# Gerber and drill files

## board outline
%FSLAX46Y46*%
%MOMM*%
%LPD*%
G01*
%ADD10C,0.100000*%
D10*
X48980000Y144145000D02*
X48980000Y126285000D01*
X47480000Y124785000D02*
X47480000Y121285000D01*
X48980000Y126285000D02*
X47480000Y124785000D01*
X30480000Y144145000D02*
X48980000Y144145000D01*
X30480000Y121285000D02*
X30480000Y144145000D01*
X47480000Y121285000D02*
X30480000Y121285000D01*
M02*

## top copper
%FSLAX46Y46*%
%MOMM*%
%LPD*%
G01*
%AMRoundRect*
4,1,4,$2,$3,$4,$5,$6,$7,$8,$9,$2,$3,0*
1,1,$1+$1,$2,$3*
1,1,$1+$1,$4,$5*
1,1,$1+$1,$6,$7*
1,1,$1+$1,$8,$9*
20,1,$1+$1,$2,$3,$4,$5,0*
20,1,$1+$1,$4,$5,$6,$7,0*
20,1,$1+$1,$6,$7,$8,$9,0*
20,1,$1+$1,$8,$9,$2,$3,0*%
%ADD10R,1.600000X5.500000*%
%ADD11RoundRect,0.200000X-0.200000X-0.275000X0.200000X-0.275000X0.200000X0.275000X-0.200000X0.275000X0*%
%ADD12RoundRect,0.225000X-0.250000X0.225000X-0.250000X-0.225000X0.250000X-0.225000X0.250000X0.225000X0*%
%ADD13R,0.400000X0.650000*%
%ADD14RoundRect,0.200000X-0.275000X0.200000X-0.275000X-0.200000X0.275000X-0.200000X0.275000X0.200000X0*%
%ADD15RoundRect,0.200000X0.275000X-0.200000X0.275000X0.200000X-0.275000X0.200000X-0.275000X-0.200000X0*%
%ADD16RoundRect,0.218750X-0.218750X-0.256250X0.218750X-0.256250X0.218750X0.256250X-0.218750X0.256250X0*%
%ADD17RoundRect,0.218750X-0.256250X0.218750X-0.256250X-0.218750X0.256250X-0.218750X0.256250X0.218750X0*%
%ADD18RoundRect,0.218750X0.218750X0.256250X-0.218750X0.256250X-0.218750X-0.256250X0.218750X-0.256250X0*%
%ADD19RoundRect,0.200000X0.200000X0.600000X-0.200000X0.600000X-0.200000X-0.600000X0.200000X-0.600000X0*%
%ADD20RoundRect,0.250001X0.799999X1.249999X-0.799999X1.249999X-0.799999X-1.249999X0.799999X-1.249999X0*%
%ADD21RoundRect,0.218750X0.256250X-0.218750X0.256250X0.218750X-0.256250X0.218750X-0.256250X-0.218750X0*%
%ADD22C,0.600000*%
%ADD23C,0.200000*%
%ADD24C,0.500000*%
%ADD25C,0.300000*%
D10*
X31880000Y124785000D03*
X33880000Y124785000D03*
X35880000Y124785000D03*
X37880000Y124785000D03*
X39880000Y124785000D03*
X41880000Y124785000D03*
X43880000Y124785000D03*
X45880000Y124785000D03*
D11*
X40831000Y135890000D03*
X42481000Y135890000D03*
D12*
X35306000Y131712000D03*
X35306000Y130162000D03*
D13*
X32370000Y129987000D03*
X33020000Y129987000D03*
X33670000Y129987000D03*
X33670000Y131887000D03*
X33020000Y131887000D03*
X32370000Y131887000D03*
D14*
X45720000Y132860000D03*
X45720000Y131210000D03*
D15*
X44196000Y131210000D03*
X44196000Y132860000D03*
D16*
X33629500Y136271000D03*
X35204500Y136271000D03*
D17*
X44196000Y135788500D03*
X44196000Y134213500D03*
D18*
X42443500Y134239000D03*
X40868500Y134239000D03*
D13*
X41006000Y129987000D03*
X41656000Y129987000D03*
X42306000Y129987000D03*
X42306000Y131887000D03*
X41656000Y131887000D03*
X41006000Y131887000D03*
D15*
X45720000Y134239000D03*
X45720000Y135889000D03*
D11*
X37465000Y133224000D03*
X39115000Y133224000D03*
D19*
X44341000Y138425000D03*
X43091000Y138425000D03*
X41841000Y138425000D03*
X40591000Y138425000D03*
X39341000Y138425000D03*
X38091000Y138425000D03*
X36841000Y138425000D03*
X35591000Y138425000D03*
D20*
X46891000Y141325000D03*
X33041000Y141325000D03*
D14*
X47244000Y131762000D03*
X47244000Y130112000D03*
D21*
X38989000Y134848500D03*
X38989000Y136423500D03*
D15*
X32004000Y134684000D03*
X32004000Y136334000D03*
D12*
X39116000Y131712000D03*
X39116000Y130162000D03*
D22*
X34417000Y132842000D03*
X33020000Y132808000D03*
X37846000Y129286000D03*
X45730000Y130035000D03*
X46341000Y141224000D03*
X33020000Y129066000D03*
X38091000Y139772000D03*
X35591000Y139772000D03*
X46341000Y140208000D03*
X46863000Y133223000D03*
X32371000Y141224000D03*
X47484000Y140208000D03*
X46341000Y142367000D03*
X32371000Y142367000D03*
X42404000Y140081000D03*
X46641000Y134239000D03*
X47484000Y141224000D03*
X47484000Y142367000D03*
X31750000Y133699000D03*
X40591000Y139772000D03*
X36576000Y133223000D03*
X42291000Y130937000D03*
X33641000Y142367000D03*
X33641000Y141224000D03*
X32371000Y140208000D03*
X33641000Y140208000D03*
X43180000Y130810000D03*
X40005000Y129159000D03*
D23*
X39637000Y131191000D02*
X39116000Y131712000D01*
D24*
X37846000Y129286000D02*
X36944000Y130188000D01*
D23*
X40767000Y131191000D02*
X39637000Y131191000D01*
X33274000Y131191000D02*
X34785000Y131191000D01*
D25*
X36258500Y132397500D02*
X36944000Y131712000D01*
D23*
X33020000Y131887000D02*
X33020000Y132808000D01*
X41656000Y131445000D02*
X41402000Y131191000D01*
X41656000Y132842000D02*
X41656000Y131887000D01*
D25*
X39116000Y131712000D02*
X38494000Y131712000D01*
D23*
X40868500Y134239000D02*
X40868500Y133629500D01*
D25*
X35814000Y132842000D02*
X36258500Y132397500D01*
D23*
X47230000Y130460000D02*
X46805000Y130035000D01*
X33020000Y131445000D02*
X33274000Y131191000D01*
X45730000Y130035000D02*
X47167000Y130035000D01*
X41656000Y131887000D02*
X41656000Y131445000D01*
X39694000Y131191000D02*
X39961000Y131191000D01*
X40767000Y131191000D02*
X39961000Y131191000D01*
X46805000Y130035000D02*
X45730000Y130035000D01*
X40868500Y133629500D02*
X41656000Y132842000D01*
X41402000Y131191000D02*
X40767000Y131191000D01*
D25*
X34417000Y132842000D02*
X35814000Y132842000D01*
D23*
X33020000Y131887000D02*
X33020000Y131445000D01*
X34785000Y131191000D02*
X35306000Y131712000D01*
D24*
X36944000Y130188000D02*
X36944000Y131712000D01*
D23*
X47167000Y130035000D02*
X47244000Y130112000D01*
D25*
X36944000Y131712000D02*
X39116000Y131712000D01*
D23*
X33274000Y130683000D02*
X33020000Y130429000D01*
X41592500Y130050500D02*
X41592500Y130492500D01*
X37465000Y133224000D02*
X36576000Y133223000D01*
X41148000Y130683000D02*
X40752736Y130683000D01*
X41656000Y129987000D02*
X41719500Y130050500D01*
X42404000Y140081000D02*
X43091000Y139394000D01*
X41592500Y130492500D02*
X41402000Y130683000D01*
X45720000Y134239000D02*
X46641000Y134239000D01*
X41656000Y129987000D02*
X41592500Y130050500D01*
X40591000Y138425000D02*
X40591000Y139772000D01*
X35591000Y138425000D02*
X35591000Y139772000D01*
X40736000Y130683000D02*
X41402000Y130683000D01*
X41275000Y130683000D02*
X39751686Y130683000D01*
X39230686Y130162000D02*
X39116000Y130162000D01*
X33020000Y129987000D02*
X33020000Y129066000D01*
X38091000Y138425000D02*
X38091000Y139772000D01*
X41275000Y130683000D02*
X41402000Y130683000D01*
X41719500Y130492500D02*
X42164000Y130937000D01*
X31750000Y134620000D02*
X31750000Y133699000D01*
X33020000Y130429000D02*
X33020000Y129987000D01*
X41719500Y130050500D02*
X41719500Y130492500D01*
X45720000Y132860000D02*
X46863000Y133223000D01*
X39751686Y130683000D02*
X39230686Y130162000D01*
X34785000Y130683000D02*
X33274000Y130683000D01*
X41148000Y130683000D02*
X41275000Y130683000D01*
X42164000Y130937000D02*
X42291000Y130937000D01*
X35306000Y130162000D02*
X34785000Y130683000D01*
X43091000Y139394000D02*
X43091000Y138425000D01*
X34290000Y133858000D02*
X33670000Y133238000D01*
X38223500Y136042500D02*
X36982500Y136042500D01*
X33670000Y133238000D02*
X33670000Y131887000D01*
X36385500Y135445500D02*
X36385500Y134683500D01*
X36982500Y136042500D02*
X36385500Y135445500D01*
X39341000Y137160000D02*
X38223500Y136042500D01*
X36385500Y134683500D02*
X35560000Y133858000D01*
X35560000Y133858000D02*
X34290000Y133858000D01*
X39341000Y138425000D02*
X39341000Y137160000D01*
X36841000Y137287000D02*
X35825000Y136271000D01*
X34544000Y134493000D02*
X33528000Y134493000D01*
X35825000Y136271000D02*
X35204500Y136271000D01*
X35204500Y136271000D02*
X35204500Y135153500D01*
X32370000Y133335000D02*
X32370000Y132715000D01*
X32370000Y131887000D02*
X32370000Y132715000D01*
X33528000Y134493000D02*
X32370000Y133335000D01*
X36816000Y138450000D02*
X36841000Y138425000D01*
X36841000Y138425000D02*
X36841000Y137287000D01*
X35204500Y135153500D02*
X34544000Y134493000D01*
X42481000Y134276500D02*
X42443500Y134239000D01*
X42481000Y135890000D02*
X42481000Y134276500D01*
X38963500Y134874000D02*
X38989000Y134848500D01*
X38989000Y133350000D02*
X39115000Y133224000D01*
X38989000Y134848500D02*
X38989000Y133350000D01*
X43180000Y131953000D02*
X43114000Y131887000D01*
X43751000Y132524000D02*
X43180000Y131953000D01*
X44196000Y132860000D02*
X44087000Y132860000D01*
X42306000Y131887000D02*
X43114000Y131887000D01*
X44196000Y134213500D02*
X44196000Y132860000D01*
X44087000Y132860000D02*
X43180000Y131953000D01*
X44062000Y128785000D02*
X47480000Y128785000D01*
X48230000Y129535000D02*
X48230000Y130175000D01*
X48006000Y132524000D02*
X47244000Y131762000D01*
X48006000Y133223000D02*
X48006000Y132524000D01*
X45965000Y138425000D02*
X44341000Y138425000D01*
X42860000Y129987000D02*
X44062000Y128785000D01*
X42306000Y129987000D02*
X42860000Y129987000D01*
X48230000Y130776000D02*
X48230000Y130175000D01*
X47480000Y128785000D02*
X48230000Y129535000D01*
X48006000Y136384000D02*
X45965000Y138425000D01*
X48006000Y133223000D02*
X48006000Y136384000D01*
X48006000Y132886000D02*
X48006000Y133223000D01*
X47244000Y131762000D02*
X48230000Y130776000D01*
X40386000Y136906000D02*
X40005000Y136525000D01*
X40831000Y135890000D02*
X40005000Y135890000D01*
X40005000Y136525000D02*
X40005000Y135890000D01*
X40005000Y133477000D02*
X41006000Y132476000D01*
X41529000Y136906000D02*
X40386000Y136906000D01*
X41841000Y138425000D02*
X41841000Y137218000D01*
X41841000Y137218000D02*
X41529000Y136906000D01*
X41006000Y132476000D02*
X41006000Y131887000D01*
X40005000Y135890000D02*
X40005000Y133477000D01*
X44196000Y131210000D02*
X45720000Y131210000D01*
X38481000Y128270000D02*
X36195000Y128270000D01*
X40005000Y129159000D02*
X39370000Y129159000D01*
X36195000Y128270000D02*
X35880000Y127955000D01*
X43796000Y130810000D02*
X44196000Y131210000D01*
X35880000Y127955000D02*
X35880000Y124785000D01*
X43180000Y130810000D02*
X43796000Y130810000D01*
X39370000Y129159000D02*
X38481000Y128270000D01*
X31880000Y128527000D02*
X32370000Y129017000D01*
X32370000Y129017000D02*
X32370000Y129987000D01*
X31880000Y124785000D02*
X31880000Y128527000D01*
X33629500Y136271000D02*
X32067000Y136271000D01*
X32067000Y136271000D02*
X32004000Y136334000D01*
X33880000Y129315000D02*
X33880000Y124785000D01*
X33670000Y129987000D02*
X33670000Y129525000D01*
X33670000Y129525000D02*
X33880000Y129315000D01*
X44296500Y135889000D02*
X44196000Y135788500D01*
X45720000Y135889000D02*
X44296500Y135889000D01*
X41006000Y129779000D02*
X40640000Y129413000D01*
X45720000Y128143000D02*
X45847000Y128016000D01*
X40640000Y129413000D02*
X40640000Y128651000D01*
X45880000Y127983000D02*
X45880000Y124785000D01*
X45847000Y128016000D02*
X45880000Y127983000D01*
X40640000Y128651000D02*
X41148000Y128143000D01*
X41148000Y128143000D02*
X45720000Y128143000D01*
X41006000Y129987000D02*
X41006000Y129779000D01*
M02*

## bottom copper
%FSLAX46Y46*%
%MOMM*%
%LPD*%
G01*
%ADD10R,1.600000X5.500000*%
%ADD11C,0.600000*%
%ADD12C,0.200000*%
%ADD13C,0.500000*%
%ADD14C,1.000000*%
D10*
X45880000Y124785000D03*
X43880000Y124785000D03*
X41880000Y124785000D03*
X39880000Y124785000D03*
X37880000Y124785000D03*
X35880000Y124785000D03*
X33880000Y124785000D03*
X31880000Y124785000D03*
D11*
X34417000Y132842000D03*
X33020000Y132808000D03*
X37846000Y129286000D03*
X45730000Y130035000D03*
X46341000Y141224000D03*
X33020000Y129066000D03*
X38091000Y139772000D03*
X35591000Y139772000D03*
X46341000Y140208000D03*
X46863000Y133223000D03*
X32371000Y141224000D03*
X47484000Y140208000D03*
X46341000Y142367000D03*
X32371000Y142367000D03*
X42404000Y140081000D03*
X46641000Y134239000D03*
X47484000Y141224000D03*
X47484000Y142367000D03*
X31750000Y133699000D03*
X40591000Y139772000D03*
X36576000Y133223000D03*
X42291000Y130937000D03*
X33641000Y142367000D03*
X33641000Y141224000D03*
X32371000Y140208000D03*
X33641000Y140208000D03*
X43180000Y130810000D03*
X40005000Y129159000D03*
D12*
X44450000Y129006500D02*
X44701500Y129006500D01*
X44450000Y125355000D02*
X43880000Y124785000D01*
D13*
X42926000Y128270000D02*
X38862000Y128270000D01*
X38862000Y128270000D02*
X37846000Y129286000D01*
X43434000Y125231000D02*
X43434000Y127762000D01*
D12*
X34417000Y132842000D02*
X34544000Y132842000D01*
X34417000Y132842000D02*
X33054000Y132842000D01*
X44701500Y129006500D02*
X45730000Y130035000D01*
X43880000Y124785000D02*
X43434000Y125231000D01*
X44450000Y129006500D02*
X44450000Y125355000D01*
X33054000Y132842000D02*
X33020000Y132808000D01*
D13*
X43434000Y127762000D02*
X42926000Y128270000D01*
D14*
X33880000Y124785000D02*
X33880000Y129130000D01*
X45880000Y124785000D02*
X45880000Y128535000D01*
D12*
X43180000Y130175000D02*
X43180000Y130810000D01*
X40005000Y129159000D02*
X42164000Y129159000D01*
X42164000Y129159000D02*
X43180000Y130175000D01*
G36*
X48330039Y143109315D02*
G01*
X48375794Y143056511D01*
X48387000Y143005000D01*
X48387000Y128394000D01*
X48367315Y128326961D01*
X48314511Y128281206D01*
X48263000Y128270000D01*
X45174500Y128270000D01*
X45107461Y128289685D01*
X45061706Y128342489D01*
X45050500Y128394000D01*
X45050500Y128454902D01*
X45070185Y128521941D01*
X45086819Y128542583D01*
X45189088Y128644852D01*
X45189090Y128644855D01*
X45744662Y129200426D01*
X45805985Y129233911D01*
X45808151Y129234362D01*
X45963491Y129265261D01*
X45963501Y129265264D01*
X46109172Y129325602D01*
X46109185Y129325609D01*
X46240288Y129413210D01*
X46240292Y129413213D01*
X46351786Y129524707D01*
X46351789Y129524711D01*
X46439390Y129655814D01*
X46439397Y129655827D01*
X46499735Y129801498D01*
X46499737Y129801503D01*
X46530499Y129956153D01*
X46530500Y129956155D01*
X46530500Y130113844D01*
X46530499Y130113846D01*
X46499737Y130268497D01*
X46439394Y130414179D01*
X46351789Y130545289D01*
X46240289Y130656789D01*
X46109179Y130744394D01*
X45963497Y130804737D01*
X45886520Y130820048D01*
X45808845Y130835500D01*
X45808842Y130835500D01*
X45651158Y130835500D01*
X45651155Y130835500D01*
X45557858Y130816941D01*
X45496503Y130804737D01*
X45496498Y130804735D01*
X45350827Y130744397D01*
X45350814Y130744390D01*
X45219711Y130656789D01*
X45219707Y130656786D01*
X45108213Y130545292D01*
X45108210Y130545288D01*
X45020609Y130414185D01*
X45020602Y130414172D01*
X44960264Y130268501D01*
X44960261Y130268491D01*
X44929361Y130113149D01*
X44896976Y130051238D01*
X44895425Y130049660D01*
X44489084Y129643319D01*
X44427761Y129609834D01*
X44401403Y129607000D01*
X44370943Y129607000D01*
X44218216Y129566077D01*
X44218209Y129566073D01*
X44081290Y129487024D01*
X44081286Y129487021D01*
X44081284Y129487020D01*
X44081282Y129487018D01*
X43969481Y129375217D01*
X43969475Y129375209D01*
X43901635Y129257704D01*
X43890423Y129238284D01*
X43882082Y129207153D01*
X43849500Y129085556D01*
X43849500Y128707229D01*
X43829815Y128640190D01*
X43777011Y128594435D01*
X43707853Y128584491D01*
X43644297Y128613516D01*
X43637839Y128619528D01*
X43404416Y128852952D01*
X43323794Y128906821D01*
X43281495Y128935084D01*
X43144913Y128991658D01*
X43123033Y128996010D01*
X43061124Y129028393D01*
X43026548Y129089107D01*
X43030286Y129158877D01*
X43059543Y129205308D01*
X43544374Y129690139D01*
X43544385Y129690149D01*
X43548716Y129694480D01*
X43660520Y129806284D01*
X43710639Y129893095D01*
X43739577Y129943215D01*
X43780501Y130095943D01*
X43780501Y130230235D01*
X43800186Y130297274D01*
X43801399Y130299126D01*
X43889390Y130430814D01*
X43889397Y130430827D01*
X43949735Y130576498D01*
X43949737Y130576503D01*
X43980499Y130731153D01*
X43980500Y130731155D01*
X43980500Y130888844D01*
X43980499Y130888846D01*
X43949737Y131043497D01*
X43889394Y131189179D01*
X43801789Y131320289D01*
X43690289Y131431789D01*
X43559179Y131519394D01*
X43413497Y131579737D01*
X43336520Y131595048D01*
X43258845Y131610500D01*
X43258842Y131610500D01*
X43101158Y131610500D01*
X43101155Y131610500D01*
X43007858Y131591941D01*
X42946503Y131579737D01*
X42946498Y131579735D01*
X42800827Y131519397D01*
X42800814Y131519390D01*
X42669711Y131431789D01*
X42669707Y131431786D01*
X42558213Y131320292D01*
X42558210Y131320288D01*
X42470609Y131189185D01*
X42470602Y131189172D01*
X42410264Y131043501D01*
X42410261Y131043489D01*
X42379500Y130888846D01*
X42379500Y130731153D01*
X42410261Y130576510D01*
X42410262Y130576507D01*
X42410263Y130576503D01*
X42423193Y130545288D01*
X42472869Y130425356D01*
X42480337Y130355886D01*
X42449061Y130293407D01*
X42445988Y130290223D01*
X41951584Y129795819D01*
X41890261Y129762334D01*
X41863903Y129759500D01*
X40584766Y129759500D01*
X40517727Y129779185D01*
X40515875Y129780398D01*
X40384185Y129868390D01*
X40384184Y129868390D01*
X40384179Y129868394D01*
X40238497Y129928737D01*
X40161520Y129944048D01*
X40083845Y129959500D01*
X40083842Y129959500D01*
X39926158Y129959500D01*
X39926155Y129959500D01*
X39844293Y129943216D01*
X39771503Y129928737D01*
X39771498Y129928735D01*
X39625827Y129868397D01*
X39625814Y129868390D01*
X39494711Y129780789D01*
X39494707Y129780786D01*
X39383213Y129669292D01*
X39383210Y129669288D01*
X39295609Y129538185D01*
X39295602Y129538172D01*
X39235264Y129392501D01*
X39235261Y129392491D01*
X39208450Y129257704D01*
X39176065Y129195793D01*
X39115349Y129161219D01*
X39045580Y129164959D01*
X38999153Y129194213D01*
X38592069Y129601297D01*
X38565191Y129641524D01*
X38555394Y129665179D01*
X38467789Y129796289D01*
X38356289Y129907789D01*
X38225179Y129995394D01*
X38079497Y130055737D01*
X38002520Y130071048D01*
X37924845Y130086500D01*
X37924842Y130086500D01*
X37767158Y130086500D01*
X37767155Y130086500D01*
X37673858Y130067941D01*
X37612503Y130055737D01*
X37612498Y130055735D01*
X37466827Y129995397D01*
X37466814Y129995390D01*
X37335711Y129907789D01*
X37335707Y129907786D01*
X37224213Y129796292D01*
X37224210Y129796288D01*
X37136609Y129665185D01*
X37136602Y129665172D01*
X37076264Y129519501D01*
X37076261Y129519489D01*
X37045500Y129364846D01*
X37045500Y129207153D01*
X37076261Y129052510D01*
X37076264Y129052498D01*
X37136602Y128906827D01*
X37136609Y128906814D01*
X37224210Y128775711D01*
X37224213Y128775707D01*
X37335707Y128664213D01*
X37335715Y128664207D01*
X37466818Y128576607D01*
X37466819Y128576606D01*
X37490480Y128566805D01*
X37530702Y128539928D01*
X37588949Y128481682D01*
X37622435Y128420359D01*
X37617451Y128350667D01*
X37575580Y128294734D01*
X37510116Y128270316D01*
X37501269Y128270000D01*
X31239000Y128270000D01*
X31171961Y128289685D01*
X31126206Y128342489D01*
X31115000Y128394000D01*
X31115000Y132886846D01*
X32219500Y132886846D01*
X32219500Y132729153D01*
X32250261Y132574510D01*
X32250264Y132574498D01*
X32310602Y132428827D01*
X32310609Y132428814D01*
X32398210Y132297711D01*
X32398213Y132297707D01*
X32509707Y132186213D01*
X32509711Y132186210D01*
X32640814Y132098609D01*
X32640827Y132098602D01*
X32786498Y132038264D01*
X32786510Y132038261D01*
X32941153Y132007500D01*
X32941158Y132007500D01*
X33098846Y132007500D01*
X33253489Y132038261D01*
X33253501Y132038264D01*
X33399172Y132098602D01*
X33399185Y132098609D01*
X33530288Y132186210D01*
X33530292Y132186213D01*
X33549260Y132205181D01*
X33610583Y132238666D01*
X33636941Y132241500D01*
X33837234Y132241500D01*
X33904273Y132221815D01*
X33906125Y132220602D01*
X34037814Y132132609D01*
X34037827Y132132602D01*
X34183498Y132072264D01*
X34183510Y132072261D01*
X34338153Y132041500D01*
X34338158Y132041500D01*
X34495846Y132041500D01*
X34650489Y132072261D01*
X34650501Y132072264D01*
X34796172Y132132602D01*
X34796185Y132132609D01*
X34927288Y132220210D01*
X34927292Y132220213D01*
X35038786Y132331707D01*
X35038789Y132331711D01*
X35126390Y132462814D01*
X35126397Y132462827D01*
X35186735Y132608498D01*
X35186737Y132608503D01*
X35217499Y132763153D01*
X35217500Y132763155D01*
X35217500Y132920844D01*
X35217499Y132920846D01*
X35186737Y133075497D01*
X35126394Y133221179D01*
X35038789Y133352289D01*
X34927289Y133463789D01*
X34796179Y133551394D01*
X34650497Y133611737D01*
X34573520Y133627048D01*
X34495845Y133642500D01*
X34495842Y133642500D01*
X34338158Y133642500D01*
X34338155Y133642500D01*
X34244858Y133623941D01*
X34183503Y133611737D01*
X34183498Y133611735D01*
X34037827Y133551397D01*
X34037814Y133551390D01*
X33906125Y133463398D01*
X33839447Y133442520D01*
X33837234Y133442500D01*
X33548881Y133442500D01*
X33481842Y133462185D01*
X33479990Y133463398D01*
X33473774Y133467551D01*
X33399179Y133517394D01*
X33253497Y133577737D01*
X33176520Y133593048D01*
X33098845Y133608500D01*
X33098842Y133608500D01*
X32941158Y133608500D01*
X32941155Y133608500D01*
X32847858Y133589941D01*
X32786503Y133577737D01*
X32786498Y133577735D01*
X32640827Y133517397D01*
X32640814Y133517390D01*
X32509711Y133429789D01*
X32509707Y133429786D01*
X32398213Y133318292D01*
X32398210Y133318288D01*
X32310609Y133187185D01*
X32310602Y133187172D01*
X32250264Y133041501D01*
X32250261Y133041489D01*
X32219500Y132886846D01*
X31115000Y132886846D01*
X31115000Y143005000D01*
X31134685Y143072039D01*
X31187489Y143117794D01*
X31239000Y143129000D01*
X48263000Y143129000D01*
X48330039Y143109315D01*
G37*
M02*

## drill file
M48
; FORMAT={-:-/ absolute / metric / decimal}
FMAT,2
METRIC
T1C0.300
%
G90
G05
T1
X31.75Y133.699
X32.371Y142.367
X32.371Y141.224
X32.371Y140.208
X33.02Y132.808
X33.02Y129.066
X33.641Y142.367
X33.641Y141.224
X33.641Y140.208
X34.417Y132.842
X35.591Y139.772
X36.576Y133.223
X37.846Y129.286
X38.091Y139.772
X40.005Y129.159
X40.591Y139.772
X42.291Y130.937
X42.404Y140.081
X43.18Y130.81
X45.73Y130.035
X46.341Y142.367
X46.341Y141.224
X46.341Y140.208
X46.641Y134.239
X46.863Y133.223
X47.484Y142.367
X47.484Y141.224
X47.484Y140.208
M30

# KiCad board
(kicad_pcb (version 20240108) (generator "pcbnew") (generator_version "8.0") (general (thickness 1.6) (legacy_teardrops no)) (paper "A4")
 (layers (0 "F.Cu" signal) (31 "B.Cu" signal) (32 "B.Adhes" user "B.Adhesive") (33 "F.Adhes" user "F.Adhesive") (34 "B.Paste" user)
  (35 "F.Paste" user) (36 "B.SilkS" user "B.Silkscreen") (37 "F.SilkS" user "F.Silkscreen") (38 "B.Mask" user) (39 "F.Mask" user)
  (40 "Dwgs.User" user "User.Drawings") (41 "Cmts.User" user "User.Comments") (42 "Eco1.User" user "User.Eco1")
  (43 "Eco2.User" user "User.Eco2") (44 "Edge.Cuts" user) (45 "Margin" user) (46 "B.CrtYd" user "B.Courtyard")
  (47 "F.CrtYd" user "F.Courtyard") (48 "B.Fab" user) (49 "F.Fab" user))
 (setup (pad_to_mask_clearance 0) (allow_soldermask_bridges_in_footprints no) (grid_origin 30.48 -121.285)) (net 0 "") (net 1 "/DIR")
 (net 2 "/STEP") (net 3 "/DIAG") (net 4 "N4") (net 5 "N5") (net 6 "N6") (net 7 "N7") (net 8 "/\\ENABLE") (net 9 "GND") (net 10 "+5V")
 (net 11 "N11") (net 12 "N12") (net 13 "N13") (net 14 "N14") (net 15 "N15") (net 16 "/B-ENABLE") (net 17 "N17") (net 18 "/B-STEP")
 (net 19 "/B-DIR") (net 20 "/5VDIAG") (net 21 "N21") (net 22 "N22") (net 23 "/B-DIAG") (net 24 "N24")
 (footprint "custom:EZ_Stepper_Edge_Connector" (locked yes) (layer "F.Cu") (at 30.48 -121.285)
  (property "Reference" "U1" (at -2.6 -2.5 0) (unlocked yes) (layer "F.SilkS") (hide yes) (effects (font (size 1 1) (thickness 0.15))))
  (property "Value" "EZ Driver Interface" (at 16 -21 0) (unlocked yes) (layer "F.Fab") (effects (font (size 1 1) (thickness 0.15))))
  (pad "1" smd rect (at 1.4 -3.5) (size 1.6 5.5) (layers "F.Cu" "F.Paste" "F.Mask") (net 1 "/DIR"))
  (pad "2" smd rect (at 3.4 -3.5) (size 1.6 5.5) (layers "F.Cu" "F.Paste" "F.Mask") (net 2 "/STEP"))
  (pad "3" smd rect (at 5.4 -3.5) (size 1.6 5.5) (layers "F.Cu" "F.Paste" "F.Mask") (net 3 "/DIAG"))
  (pad "4" smd rect (at 7.4 -3.5) (size 1.6 5.5) (layers "F.Cu" "F.Paste" "F.Mask") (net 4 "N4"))
  (pad "5" smd rect (at 9.4 -3.5) (size 1.6 5.5) (layers "F.Cu" "F.Paste" "F.Mask") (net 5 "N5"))
  (pad "6" smd rect (at 11.4 -3.5) (size 1.6 5.5) (layers "F.Cu" "F.Paste" "F.Mask") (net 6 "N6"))
  (pad "7" smd rect (at 13.4 -3.5) (size 1.6 5.5) (layers "F.Cu" "F.Paste" "F.Mask") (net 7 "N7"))
  (pad "8" smd rect (at 15.4 -3.5) (size 1.6 5.5) (layers "F.Cu" "F.Paste" "F.Mask") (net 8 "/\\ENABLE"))
  (pad "9" smd rect (at 15.4 -3.5) (size 1.6 5.5) (layers "B.Cu" "B.Paste" "B.Mask") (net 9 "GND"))
  (pad "10" smd rect (at 13.4 -3.5) (size 1.6 5.5) (layers "B.Cu" "B.Paste" "B.Mask") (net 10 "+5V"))
  (pad "11" smd rect (at 11.4 -3.5) (size 1.6 5.5) (layers "B.Cu" "B.Paste" "B.Mask") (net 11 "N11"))
  (pad "12" smd rect (at 9.4 -3.5) (size 1.6 5.5) (layers "B.Cu" "B.Paste" "B.Mask") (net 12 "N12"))
  (pad "13" smd rect (at 7.4 -3.5) (size 1.6 5.5) (layers "B.Cu" "B.Paste" "B.Mask") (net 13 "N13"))
  (pad "14" smd rect (at 5.4 -3.5) (size 1.6 5.5) (layers "B.Cu" "B.Paste" "B.Mask") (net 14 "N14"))
  (pad "15" smd rect (at 3.4 -3.5) (size 1.6 5.5) (layers "B.Cu" "B.Paste" "B.Mask") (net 9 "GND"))
  (pad "16" smd rect (at 1.4 -3.5) (size 1.6 5.5) (layers "B.Cu" "B.Paste" "B.Mask") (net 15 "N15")))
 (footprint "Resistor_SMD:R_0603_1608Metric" (layer "F.Cu") (at 41.656 -135.89)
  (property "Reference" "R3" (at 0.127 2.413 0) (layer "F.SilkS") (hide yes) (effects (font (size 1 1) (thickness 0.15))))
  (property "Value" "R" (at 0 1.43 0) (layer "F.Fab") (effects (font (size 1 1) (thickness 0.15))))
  (pad "1" smd roundrect (at -0.825 0) (size 0.8 0.95) (layers "F.Cu" "F.Paste" "F.Mask") (roundrect_rratio 0.25) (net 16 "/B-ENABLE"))
  (pad "2" smd roundrect (at 0.825 0) (size 0.8 0.95) (layers "F.Cu" "F.Paste" "F.Mask") (roundrect_rratio 0.25) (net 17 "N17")))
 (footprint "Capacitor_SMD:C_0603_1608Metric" (layer "F.Cu") (at 35.306 -130.937 -90)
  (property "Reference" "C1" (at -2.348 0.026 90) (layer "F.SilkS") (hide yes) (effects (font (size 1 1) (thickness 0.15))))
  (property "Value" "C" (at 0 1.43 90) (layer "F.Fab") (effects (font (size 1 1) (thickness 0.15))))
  (pad "1" smd roundrect (at -0.775 0 270) (size 0.9 0.95) (layers "F.Cu" "F.Paste" "F.Mask") (roundrect_rratio 0.25) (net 10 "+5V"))
  (pad "2" smd roundrect (at 0.775 0 270) (size 0.9 0.95) (layers "F.Cu" "F.Paste" "F.Mask") (roundrect_rratio 0.25) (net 9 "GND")))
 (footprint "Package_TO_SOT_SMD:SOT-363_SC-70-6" (layer "F.Cu") (at 33.02 -130.937 90)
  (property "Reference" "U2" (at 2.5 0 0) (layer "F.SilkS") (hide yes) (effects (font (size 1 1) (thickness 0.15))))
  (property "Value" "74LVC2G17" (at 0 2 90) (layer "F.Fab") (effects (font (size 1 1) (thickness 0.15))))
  (pad "1" smd rect (at -0.95 -0.65 90) (size 0.65 0.4) (layers "F.Cu" "F.Paste" "F.Mask") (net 1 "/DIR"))
  (pad "2" smd rect (at -0.95 0 90) (size 0.65 0.4) (layers "F.Cu" "F.Paste" "F.Mask") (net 9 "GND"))
  (pad "3" smd rect (at -0.95 0.65 90) (size 0.65 0.4) (layers "F.Cu" "F.Paste" "F.Mask") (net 2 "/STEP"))
  (pad "4" smd rect (at 0.95 0.65 90) (size 0.65 0.4) (layers "F.Cu" "F.Paste" "F.Mask") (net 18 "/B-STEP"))
  (pad "5" smd rect (at 0.95 0 90) (size 0.65 0.4) (layers "F.Cu" "F.Paste" "F.Mask") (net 10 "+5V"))
  (pad "6" smd rect (at 0.95 -0.65 90) (size 0.65 0.4) (layers "F.Cu" "F.Paste" "F.Mask") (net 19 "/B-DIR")))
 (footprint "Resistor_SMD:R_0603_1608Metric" (layer "F.Cu") (at 45.72 -132.035 -90)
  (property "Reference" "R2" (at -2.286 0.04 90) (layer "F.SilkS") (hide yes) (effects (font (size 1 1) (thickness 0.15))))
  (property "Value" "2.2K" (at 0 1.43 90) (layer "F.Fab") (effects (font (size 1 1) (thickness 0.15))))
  (pad "1" smd roundrect (at -0.825 0 270) (size 0.8 0.95) (layers "F.Cu" "F.Paste" "F.Mask") (roundrect_rratio 0.25) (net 9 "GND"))
  (pad "2" smd roundrect (at 0.825 0 270) (size 0.8 0.95) (layers "F.Cu" "F.Paste" "F.Mask") (roundrect_rratio 0.25) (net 3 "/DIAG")))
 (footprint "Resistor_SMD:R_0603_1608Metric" (layer "F.Cu") (at 44.196 -132.035 90)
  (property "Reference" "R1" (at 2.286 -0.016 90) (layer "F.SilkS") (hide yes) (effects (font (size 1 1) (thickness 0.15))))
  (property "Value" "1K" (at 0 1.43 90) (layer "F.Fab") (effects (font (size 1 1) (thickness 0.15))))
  (pad "1" smd roundrect (at -0.825 0 90) (size 0.8 0.95) (layers "F.Cu" "F.Paste" "F.Mask") (roundrect_rratio 0.25) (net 3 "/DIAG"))
  (pad "2" smd roundrect (at 0.825 0 90) (size 0.8 0.95) (layers "F.Cu" "F.Paste" "F.Mask") (roundrect_rratio 0.25) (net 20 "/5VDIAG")))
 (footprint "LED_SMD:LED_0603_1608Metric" (layer "F.Cu") (at 34.417 -136.271)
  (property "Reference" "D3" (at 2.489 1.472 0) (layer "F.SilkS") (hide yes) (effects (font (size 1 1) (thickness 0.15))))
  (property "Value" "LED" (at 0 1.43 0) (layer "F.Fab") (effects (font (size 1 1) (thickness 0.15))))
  (pad "1" smd roundrect (at -0.7875 0) (size 0.875 0.95) (layers "F.Cu" "F.Paste" "F.Mask") (roundrect_rratio 0.25) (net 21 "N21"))
  (pad "2" smd roundrect (at 0.7875 0) (size 0.875 0.95) (layers "F.Cu" "F.Paste" "F.Mask") (roundrect_rratio 0.25) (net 19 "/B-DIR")))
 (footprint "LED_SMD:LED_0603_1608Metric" (layer "F.Cu") (at 44.196 -135.001 -90)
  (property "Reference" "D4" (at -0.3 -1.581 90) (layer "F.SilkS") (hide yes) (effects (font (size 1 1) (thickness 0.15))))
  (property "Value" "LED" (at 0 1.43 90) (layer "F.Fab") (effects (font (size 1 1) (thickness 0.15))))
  (pad "1" smd roundrect (at -0.7875 0 270) (size 0.875 0.95) (layers "F.Cu" "F.Paste" "F.Mask") (roundrect_rratio 0.25) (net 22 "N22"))
  (pad "2" smd roundrect (at 0.7875 0 270) (size 0.875 0.95) (layers "F.Cu" "F.Paste" "F.Mask") (roundrect_rratio 0.25) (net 20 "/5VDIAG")))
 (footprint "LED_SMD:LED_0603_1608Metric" (layer "F.Cu") (at 41.656 -134.239 180)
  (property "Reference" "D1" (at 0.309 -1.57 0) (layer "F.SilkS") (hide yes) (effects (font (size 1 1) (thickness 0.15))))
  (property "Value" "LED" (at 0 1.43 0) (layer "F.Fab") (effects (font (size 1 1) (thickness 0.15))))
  (pad "1" smd roundrect (at -0.7875 0 180) (size 0.875 0.95) (layers "F.Cu" "F.Paste" "F.Mask") (roundrect_rratio 0.25) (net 17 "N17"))
  (pad "2" smd roundrect (at 0.7875 0 180) (size 0.875 0.95) (layers "F.Cu" "F.Paste" "F.Mask") (roundrect_rratio 0.25) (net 10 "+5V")))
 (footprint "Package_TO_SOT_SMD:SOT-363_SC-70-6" (layer "F.Cu") (at 41.656 -130.937 90)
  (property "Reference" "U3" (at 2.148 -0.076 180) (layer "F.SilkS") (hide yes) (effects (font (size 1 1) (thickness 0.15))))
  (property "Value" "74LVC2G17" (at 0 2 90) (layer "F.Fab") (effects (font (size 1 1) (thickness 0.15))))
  (pad "1" smd rect (at -0.95 -0.65 90) (size 0.65 0.4) (layers "F.Cu" "F.Paste" "F.Mask") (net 8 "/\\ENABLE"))
  (pad "2" smd rect (at -0.95 0 90) (size 0.65 0.4) (layers "F.Cu" "F.Paste" "F.Mask") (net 9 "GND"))
  (pad "3" smd rect (at -0.95 0.65 90) (size 0.65 0.4) (layers "F.Cu" "F.Paste" "F.Mask") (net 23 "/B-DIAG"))
  (pad "4" smd rect (at 0.95 0.65 90) (size 0.65 0.4) (layers "F.Cu" "F.Paste" "F.Mask") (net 20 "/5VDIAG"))
  (pad "5" smd rect (at 0.95 0 90) (size 0.65 0.4) (layers "F.Cu" "F.Paste" "F.Mask") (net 10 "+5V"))
  (pad "6" smd rect (at 0.95 -0.65 90) (size 0.65 0.4) (layers "F.Cu" "F.Paste" "F.Mask") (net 16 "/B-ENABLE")))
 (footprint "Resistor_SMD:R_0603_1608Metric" (layer "F.Cu") (at 45.72 -135.064 90)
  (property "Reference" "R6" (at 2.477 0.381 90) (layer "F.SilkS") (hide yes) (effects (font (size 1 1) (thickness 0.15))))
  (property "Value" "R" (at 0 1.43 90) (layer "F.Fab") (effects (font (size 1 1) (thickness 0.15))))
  (pad "1" smd roundrect (at -0.825 0 90) (size 0.8 0.95) (layers "F.Cu" "F.Paste" "F.Mask") (roundrect_rratio 0.25) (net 9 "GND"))
  (pad "2" smd roundrect (at 0.825 0 90) (size 0.8 0.95) (layers "F.Cu" "F.Paste" "F.Mask") (roundrect_rratio 0.25) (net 22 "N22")))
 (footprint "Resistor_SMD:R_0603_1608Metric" (layer "F.Cu") (at 38.29 -133.224)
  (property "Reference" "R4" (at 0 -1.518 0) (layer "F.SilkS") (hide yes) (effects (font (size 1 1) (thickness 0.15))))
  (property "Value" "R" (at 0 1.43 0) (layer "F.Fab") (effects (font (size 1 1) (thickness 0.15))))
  (pad "1" smd roundrect (at -0.825 0) (size 0.8 0.95) (layers "F.Cu" "F.Paste" "F.Mask") (roundrect_rratio 0.25) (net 9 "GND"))
  (pad "2" smd roundrect (at 0.825 0) (size 0.8 0.95) (layers "F.Cu" "F.Paste" "F.Mask") (roundrect_rratio 0.25) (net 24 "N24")))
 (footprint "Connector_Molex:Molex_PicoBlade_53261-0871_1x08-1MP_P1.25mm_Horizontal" (layer "F.Cu") (at 39.966 -140.825 180)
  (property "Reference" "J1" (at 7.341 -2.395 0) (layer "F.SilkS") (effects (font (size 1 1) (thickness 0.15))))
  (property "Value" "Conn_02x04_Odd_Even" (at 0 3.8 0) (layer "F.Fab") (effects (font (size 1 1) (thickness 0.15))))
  (pad "1" smd roundrect (at -4.375 -2.4 180) (size 0.8 1.6) (layers "F.Cu" "F.Paste" "F.Mask") (roundrect_rratio 0.25) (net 23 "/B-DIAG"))
  (pad "2" smd roundrect (at -3.125 -2.4 180) (size 0.8 1.6) (layers "F.Cu" "F.Paste" "F.Mask") (roundrect_rratio 0.25) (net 9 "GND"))
  (pad "3" smd roundrect (at -1.875 -2.4 180) (size 0.8 1.6) (layers "F.Cu" "F.Paste" "F.Mask") (roundrect_rratio 0.25) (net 16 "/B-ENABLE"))
  (pad "4" smd roundrect (at -0.625 -2.4 180) (size 0.8 1.6) (layers "F.Cu" "F.Paste" "F.Mask") (roundrect_rratio 0.25) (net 9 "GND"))
  (pad "5" smd roundrect (at 0.625 -2.4 180) (size 0.8 1.6) (layers "F.Cu" "F.Paste" "F.Mask") (roundrect_rratio 0.25) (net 18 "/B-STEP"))
  (pad "6" smd roundrect (at 1.875 -2.4 180) (size 0.8 1.6) (layers "F.Cu" "F.Paste" "F.Mask") (roundrect_rratio 0.25) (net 9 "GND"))
  (pad "7" smd roundrect (at 3.125 -2.4 180) (size 0.8 1.6) (layers "F.Cu" "F.Paste" "F.Mask") (roundrect_rratio 0.25) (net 19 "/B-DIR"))
  (pad "8" smd roundrect (at 4.375 -2.4 180) (size 0.8 1.6) (layers "F.Cu" "F.Paste" "F.Mask") (roundrect_rratio 0.25) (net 9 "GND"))
  (pad "MP" smd roundrect (at -6.925 0.5 180) (size 2.1 3) (layers "F.Cu" "F.Paste" "F.Mask") (roundrect_rratio 0.1190480952) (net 9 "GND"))
  (pad "MP" smd roundrect (at 6.925 0.5 180) (size 2.1 3) (layers "F.Cu" "F.Paste" "F.Mask") (roundrect_rratio 0.1190480952) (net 9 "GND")))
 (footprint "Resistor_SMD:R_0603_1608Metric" (layer "F.Cu") (at 47.244 -130.937 -90)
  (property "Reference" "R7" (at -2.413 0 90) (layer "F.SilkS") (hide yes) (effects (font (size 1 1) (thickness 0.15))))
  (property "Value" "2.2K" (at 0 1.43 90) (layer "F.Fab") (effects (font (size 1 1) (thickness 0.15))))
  (pad "1" smd roundrect (at -0.825 0 270) (size 0.8 0.95) (layers "F.Cu" "F.Paste" "F.Mask") (roundrect_rratio 0.25) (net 23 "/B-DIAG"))
  (pad "2" smd roundrect (at 0.825 0 270) (size 0.8 0.95) (layers "F.Cu" "F.Paste" "F.Mask") (roundrect_rratio 0.25) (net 10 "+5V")))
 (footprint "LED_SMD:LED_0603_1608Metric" (layer "F.Cu") (at 38.989 -135.636 90)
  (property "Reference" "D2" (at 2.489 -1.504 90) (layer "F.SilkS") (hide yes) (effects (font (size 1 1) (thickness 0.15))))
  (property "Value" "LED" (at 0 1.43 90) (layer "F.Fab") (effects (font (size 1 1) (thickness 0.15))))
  (pad "1" smd roundrect (at -0.7875 0 90) (size 0.875 0.95) (layers "F.Cu" "F.Paste" "F.Mask") (roundrect_rratio 0.25) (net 24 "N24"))
  (pad "2" smd roundrect (at 0.7875 0 90) (size 0.875 0.95) (layers "F.Cu" "F.Paste" "F.Mask") (roundrect_rratio 0.25) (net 18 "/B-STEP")))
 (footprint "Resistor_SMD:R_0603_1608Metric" (layer "F.Cu") (at 32.004 -135.509 90)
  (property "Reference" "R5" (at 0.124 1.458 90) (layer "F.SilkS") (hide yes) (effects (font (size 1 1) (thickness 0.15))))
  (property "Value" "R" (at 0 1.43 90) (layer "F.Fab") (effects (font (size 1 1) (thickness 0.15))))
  (pad "1" smd roundrect (at -0.825 0 90) (size 0.8 0.95) (layers "F.Cu" "F.Paste" "F.Mask") (roundrect_rratio 0.25) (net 9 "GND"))
  (pad "2" smd roundrect (at 0.825 0 90) (size 0.8 0.95) (layers "F.Cu" "F.Paste" "F.Mask") (roundrect_rratio 0.25) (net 21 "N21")))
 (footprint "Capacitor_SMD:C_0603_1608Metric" (layer "F.Cu") (at 39.116 -130.937 -90)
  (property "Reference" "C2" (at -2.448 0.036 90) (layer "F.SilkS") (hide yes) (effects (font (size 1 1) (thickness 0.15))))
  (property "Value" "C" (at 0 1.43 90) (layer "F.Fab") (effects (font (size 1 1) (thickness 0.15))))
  (pad "1" smd roundrect (at -0.775 0 270) (size 0.9 0.95) (layers "F.Cu" "F.Paste" "F.Mask") (roundrect_rratio 0.25) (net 10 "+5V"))
  (pad "2" smd roundrect (at 0.775 0 270) (size 0.9 0.95) (layers "F.Cu" "F.Paste" "F.Mask") (roundrect_rratio 0.25) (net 9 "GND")))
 (gr_line (start 48.98 -144.145) (end 48.98 -126.285) (stroke (width 0.1) (type default)) (layer "Edge.Cuts"))
 (gr_line (start 47.48 -124.785) (end 47.48 -121.285) (stroke (width 0.1) (type default)) (layer "Edge.Cuts"))
 (gr_line (start 48.98 -126.285) (end 47.48 -124.785) (stroke (width 0.1) (type default)) (layer "Edge.Cuts"))
 (gr_line (start 30.48 -144.145) (end 48.98 -144.145) (stroke (width 0.1) (type default)) (layer "Edge.Cuts"))
 (gr_line (start 30.48 -121.285) (end 30.48 -144.145) (stroke (width 0.1) (type default)) (layer "Edge.Cuts"))
 (gr_line (start 47.48 -121.285) (end 30.48 -121.285) (stroke (width 0.1) (type default)) (layer "Edge.Cuts"))
 (segment (start 39.637 -131.191) (end 39.116 -131.712) (width 0.2) (layer "F.Cu") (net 10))
 (segment (start 37.846 -129.286) (end 36.944 -130.188) (width 0.5) (layer "F.Cu") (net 10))
 (segment (start 40.767 -131.191) (end 39.637 -131.191) (width 0.2) (layer "F.Cu") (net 10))
 (segment (start 33.274 -131.191) (end 34.785 -131.191) (width 0.2) (layer "F.Cu") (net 10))
 (segment (start 36.2585 -132.3975) (end 36.944 -131.712) (width 0.3) (layer "F.Cu") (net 10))
 (segment (start 33.02 -131.887) (end 33.02 -132.808) (width 0.2) (layer "F.Cu") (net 10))
 (segment (start 41.656 -131.445) (end 41.402 -131.191) (width 0.2) (layer "F.Cu") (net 10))
 (segment (start 41.656 -132.842) (end 41.656 -131.887) (width 0.2) (layer "F.Cu") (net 10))
 (segment (start 39.116 -131.712) (end 38.494 -131.712) (width 0.3) (layer "F.Cu") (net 10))
 (segment (start 40.8685 -134.239) (end 40.8685 -133.6295) (width 0.2) (layer "F.Cu") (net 10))
 (segment (start 35.814 -132.842) (end 36.2585 -132.3975) (width 0.3) (layer "F.Cu") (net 10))
 (segment (start 47.23 -130.46) (end 46.805 -130.035) (width 0.2) (layer "F.Cu") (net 10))
 (segment (start 33.02 -131.445) (end 33.274 -131.191) (width 0.2) (layer "F.Cu") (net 10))
 (segment (start 45.73 -130.035) (end 47.167 -130.035) (width 0.2) (layer "F.Cu") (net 10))
 (segment (start 41.656 -131.887) (end 41.656 -131.445) (width 0.2) (layer "F.Cu") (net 10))
 (segment (start 39.694 -131.191) (end 39.961 -131.191) (width 0.2) (layer "F.Cu") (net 10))
 (segment (start 40.767 -131.191) (end 39.961 -131.191) (width 0.2) (layer "F.Cu") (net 10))
 (segment (start 46.805 -130.035) (end 45.73 -130.035) (width 0.2) (layer "F.Cu") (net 10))
 (segment (start 40.8685 -133.6295) (end 41.656 -132.842) (width 0.2) (layer "F.Cu") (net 10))
 (segment (start 41.402 -131.191) (end 40.767 -131.191) (width 0.2) (layer "F.Cu") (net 10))
 (segment (start 34.417 -132.842) (end 35.814 -132.842) (width 0.3) (layer "F.Cu") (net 10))
 (segment (start 33.02 -131.887) (end 33.02 -131.445) (width 0.2) (layer "F.Cu") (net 10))
 (segment (start 34.785 -131.191) (end 35.306 -131.712) (width 0.2) (layer "F.Cu") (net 10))
 (segment (start 36.944 -130.188) (end 36.944 -131.712) (width 0.5) (layer "F.Cu") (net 10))
 (segment (start 47.167 -130.035) (end 47.244 -130.112) (width 0.2) (layer "F.Cu") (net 10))
 (segment (start 36.944 -131.712) (end 39.116 -131.712) (width 0.3) (layer "F.Cu") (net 10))
 (via (at 34.417 -132.842) (size 0.6) (drill 0.3) (layers "F.Cu" "B.Cu") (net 10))
 (via (at 33.02 -132.808) (size 0.6) (drill 0.3) (layers "F.Cu" "B.Cu") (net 10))
 (via (at 37.846 -129.286) (size 0.6) (drill 0.3) (layers "F.Cu" "B.Cu") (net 10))
 (via (at 45.73 -130.035) (size 0.6) (drill 0.3) (layers "F.Cu" "B.Cu") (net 10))
 (segment (start 44.45 -129.0065) (end 44.7015 -129.0065) (width 0.2) (layer "B.Cu") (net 10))
 (segment (start 44.45 -125.355) (end 43.88 -124.785) (width 0.2) (layer "B.Cu") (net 10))
 (segment (start 42.926 -128.27) (end 38.862 -128.27) (width 0.5) (layer "B.Cu") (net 10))
 (segment (start 38.862 -128.27) (end 37.846 -129.286) (width 0.5) (layer "B.Cu") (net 10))
 (segment (start 43.434 -125.231) (end 43.434 -127.762) (width 0.5) (layer "B.Cu") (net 10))
 (segment (start 34.417 -132.842) (end 34.544 -132.842) (width 0.2) (layer "B.Cu") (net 10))
 (segment (start 34.417 -132.842) (end 33.054 -132.842) (width 0.2) (layer "B.Cu") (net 10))
 (segment (start 44.7015 -129.0065) (end 45.73 -130.035) (width 0.2) (layer "B.Cu") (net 10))
 (segment (start 43.88 -124.785) (end 43.434 -125.231) (width 0.2) (layer "B.Cu") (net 10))
 (segment (start 44.45 -129.0065) (end 44.45 -125.355) (width 0.2) (layer "B.Cu") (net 10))
 (segment (start 33.054 -132.842) (end 33.02 -132.808) (width 0.2) (layer "B.Cu") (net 10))
 (segment (start 43.434 -127.762) (end 42.926 -128.27) (width 0.5) (layer "B.Cu") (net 10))
 (segment (start 33.274 -130.683) (end 33.02 -130.429) (width 0.2) (layer "F.Cu") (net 9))
 (segment (start 41.5925 -130.0505) (end 41.5925 -130.4925) (width 0.2) (layer "F.Cu") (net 9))
 (segment (start 37.465 -133.224) (end 36.576 -133.223) (width 0.2) (layer "F.Cu") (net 9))
 (segment (start 41.148 -130.683) (end 40.752736 -130.683) (width 0.2) (layer "F.Cu") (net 9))
 (segment (start 41.656 -129.987) (end 41.7195 -130.0505) (width 0.2) (layer "F.Cu") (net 9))
 (segment (start 42.404 -140.081) (end 43.091 -139.394) (width 0.2) (layer "F.Cu") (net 9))
 (segment (start 41.5925 -130.4925) (end 41.402 -130.683) (width 0.2) (layer "F.Cu") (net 9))
 (segment (start 45.72 -134.239) (end 46.641 -134.239) (width 0.2) (layer "F.Cu") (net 9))
 (segment (start 41.656 -129.987) (end 41.5925 -130.0505) (width 0.2) (layer "F.Cu") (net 9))
 (segment (start 40.591 -138.425) (end 40.591 -139.772) (width 0.2) (layer "F.Cu") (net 9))
 (segment (start 35.591 -138.425) (end 35.591 -139.772) (width 0.2) (layer "F.Cu") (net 9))
 (segment (start 40.736 -130.683) (end 41.402 -130.683) (width 0.2) (layer "F.Cu") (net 9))
 (segment (start 41.275 -130.683) (end 39.751686 -130.683) (width 0.2) (layer "F.Cu") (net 9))
 (segment (start 39.230686 -130.162) (end 39.116 -130.162) (width 0.2) (layer "F.Cu") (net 9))
 (segment (start 33.02 -129.987) (end 33.02 -129.066) (width 0.2) (layer "F.Cu") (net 9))
 (segment (start 38.091 -138.425) (end 38.091 -139.772) (width 0.2) (layer "F.Cu") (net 9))
 (segment (start 41.275 -130.683) (end 41.402 -130.683) (width 0.2) (layer "F.Cu") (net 9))
 (segment (start 41.7195 -130.4925) (end 42.164 -130.937) (width 0.2) (layer "F.Cu") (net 9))
 (segment (start 31.75 -134.62) (end 31.75 -133.699) (width 0.2) (layer "F.Cu") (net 9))
 (segment (start 33.02 -130.429) (end 33.02 -129.987) (width 0.2) (layer "F.Cu") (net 9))
 (segment (start 41.7195 -130.0505) (end 41.7195 -130.4925) (width 0.2) (layer "F.Cu") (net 9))
 (segment (start 45.72 -132.86) (end 46.863 -133.223) (width 0.2) (layer "F.Cu") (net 9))
 (segment (start 39.751686 -130.683) (end 39.230686 -130.162) (width 0.2) (layer "F.Cu") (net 9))
 (segment (start 34.785 -130.683) (end 33.274 -130.683) (width 0.2) (layer "F.Cu") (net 9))
 (segment (start 41.148 -130.683) (end 41.275 -130.683) (width 0.2) (layer "F.Cu") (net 9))
 (segment (start 42.164 -130.937) (end 42.291 -130.937) (width 0.2) (layer "F.Cu") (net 9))
 (segment (start 35.306 -130.162) (end 34.785 -130.683) (width 0.2) (layer "F.Cu") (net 9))
 (segment (start 43.091 -139.394) (end 43.091 -138.425) (width 0.2) (layer "F.Cu") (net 9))
 (via (at 46.341 -141.224) (size 0.6) (drill 0.3) (layers "F.Cu" "B.Cu") (free yes) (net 9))
 (via (at 33.02 -129.066) (size 0.6) (drill 0.3) (layers "F.Cu" "B.Cu") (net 9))
 (via (at 38.091 -139.772) (size 0.6) (drill 0.3) (layers "F.Cu" "B.Cu") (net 9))
 (via (at 35.591 -139.772) (size 0.6) (drill 0.3) (layers "F.Cu" "B.Cu") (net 9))
 (via (at 46.341 -140.208) (size 0.6) (drill 0.3) (layers "F.Cu" "B.Cu") (free yes) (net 9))
 (via (at 46.863 -133.223) (size 0.6) (drill 0.3) (layers "F.Cu" "B.Cu") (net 9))
 (via (at 32.371 -141.224) (size 0.6) (drill 0.3) (layers "F.Cu" "B.Cu") (free yes) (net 9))
 (via (at 47.484 -140.208) (size 0.6) (drill 0.3) (layers "F.Cu" "B.Cu") (free yes) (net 9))
 (via (at 46.341 -142.367) (size 0.6) (drill 0.3) (layers "F.Cu" "B.Cu") (free yes) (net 9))
 (via (at 32.371 -142.367) (size 0.6) (drill 0.3) (layers "F.Cu" "B.Cu") (free yes) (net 9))
 (via (at 42.404 -140.081) (size 0.6) (drill 0.3) (layers "F.Cu" "B.Cu") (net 9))
 (via (at 46.641 -134.239) (size 0.6) (drill 0.3) (layers "F.Cu" "B.Cu") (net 9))
 (via (at 47.484 -141.224) (size 0.6) (drill 0.3) (layers "F.Cu" "B.Cu") (free yes) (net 9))
 (via (at 47.484 -142.367) (size 0.6) (drill 0.3) (layers "F.Cu" "B.Cu") (free yes) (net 9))
 (via (at 31.75 -133.699) (size 0.6) (drill 0.3) (layers "F.Cu" "B.Cu") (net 9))
 (via (at 40.591 -139.772) (size 0.6) (drill 0.3) (layers "F.Cu" "B.Cu") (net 9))
 (via (at 36.576 -133.223) (size 0.6) (drill 0.3) (layers "F.Cu" "B.Cu") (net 9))
 (via (at 42.291 -130.937) (size 0.6) (drill 0.3) (layers "F.Cu" "B.Cu") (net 9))
 (via (at 33.641 -142.367) (size 0.6) (drill 0.3) (layers "F.Cu" "B.Cu") (free yes) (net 9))
 (via (at 33.641 -141.224) (size 0.6) (drill 0.3) (layers "F.Cu" "B.Cu") (free yes) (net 9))
 (via (at 32.371 -140.208) (size 0.6) (drill 0.3) (layers "F.Cu" "B.Cu") (free yes) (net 9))
 (via (at 33.641 -140.208) (size 0.6) (drill 0.3) (layers "F.Cu" "B.Cu") (free yes) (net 9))
 (segment (start 33.88 -124.785) (end 33.88 -129.13) (width 1) (layer "B.Cu") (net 9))
 (segment (start 45.88 -124.785) (end 45.88 -128.535) (width 1) (layer "B.Cu") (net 9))
 (segment (start 34.29 -133.858) (end 33.67 -133.238) (width 0.2) (layer "F.Cu") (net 18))
 (segment (start 38.2235 -136.0425) (end 36.9825 -136.0425) (width 0.2) (layer "F.Cu") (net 18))
 (segment (start 33.67 -133.238) (end 33.67 -131.887) (width 0.2) (layer "F.Cu") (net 18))
 (segment (start 36.3855 -135.4455) (end 36.3855 -134.6835) (width 0.2) (layer "F.Cu") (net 18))
 (segment (start 36.9825 -136.0425) (end 36.3855 -135.4455) (width 0.2) (layer "F.Cu") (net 18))
 (segment (start 39.341 -137.16) (end 38.2235 -136.0425) (width 0.2) (layer "F.Cu") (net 18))
 (segment (start 36.3855 -134.6835) (end 35.56 -133.858) (width 0.2) (layer "F.Cu") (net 18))
 (segment (start 35.56 -133.858) (end 34.29 -133.858) (width 0.2) (layer "F.Cu") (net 18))
 (segment (start 39.341 -138.425) (end 39.341 -137.16) (width 0.2) (layer "F.Cu") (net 18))
 (segment (start 36.841 -137.287) (end 35.825 -136.271) (width 0.2) (layer "F.Cu") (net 19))
 (segment (start 34.544 -134.493) (end 33.528 -134.493) (width 0.2) (layer "F.Cu") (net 19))
 (segment (start 35.825 -136.271) (end 35.2045 -136.271) (width 0.2) (layer "F.Cu") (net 19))
 (segment (start 35.2045 -136.271) (end 35.2045 -135.1535) (width 0.2) (layer "F.Cu") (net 19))
 (segment (start 32.37 -133.335) (end 32.37 -132.715) (width 0.2) (layer "F.Cu") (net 19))
 (segment (start 32.37 -131.887) (end 32.37 -132.715) (width 0.2) (layer "F.Cu") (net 19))
 (segment (start 33.528 -134.493) (end 32.37 -133.335) (width 0.2) (layer "F.Cu") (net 19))
 (segment (start 36.816 -138.45) (end 36.841 -138.425) (width 0.2) (layer "F.Cu") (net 19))
 (segment (start 36.841 -138.425) (end 36.841 -137.287) (width 0.2) (layer "F.Cu") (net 19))
 (segment (start 35.2045 -135.1535) (end 34.544 -134.493) (width 0.2) (layer "F.Cu") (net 19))
 (segment (start 42.481 -134.2765) (end 42.4435 -134.239) (width 0.2) (layer "F.Cu") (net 17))
 (segment (start 42.481 -135.89) (end 42.481 -134.2765) (width 0.2) (layer "F.Cu") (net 17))
 (segment (start 38.9635 -134.874) (end 38.989 -134.8485) (width 0.2) (layer "F.Cu") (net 24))
 (segment (start 38.989 -133.35) (end 39.115 -133.224) (width 0.2) (layer "F.Cu") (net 24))
 (segment (start 38.989 -134.8485) (end 38.989 -133.35) (width 0.2) (layer "F.Cu") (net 24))
 (segment (start 43.18 -131.953) (end 43.114 -131.887) (width 0.2) (layer "F.Cu") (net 20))
 (segment (start 43.751 -132.524) (end 43.18 -131.953) (width 0.2) (layer "F.Cu") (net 20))
 (segment (start 44.196 -132.86) (end 44.087 -132.86) (width 0.2) (layer "F.Cu") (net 20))
 (segment (start 42.306 -131.887) (end 43.114 -131.887) (width 0.2) (layer "F.Cu") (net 20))
 (segment (start 44.196 -134.2135) (end 44.196 -132.86) (width 0.2) (layer "F.Cu") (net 20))
 (segment (start 44.087 -132.86) (end 43.18 -131.953) (width 0.2) (layer "F.Cu") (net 20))
 (segment (start 44.062 -128.785) (end 47.48 -128.785) (width 0.2) (layer "F.Cu") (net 23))
 (segment (start 48.23 -129.535) (end 48.23 -130.175) (width 0.2) (layer "F.Cu") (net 23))
 (segment (start 48.006 -132.524) (end 47.244 -131.762) (width 0.2) (layer "F.Cu") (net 23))
 (segment (start 48.006 -133.223) (end 48.006 -132.524) (width 0.2) (layer "F.Cu") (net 23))
 (segment (start 45.965 -138.425) (end 44.341 -138.425) (width 0.2) (layer "F.Cu") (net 23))
 (segment (start 42.86 -129.987) (end 44.062 -128.785) (width 0.2) (layer "F.Cu") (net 23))
 (segment (start 42.306 -129.987) (end 42.86 -129.987) (width 0.2) (layer "F.Cu") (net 23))
 (segment (start 48.23 -130.776) (end 48.23 -130.175) (width 0.2) (layer "F.Cu") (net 23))
 (segment (start 47.48 -128.785) (end 48.23 -129.535) (width 0.2) (layer "F.Cu") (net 23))
 (segment (start 48.006 -136.384) (end 45.965 -138.425) (width 0.2) (layer "F.Cu") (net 23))
 (segment (start 48.006 -133.223) (end 48.006 -136.384) (width 0.2) (layer "F.Cu") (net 23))
 (segment (start 48.006 -132.886) (end 48.006 -133.223) (width 0.2) (layer "F.Cu") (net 23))
 (segment (start 47.244 -131.762) (end 48.23 -130.776) (width 0.2) (layer "F.Cu") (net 23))
 (segment (start 40.386 -136.906) (end 40.005 -136.525) (width 0.2) (layer "F.Cu") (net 16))
 (segment (start 40.831 -135.89) (end 40.005 -135.89) (width 0.2) (layer "F.Cu") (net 16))
 (segment (start 40.005 -136.525) (end 40.005 -135.89) (width 0.2) (layer "F.Cu") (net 16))
 (segment (start 40.005 -133.477) (end 41.006 -132.476) (width 0.2) (layer "F.Cu") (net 16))
 (segment (start 41.529 -136.906) (end 40.386 -136.906) (width 0.2) (layer "F.Cu") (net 16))
 (segment (start 41.841 -138.425) (end 41.841 -137.218) (width 0.2) (layer "F.Cu") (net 16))
 (segment (start 41.841 -137.218) (end 41.529 -136.906) (width 0.2) (layer "F.Cu") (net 16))
 (segment (start 41.006 -132.476) (end 41.006 -131.887) (width 0.2) (layer "F.Cu") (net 16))
 (segment (start 40.005 -135.89) (end 40.005 -133.477) (width 0.2) (layer "F.Cu") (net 16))
 (segment (start 44.196 -131.21) (end 45.72 -131.21) (width 0.2) (layer "F.Cu") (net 3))
 (segment (start 38.481 -128.27) (end 36.195 -128.27) (width 0.2) (layer "F.Cu") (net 3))
 (segment (start 40.005 -129.159) (end 39.37 -129.159) (width 0.2) (layer "F.Cu") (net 3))
 (segment (start 36.195 -128.27) (end 35.88 -127.955) (width 0.2) (layer "F.Cu") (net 3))
 (segment (start 43.796 -130.81) (end 44.196 -131.21) (width 0.2) (layer "F.Cu") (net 3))
 (segment (start 35.88 -127.955) (end 35.88 -124.785) (width 0.2) (layer "F.Cu") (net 3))
 (segment (start 43.18 -130.81) (end 43.796 -130.81) (width 0.2) (layer "F.Cu") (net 3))
 (segment (start 39.37 -129.159) (end 38.481 -128.27) (width 0.2) (layer "F.Cu") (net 3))
 (via (at 43.18 -130.81) (size 0.6) (drill 0.3) (layers "F.Cu" "B.Cu") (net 3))
 (via (at 40.005 -129.159) (size 0.6) (drill 0.3) (layers "F.Cu" "B.Cu") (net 3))
 (segment (start 43.18 -130.175) (end 43.18 -130.81) (width 0.2) (layer "B.Cu") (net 3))
 (segment (start 40.005 -129.159) (end 42.164 -129.159) (width 0.2) (layer "B.Cu") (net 3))
 (segment (start 42.164 -129.159) (end 43.18 -130.175) (width 0.2) (layer "B.Cu") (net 3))
 (segment (start 31.88 -128.527) (end 32.37 -129.017) (width 0.2) (layer "F.Cu") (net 1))
 (segment (start 32.37 -129.017) (end 32.37 -129.987) (width 0.2) (layer "F.Cu") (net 1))
 (segment (start 31.88 -124.785) (end 31.88 -128.527) (width 0.2) (layer "F.Cu") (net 1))
 (segment (start 33.6295 -136.271) (end 32.067 -136.271) (width 0.2) (layer "F.Cu") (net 21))
 (segment (start 32.067 -136.271) (end 32.004 -136.334) (width 0.2) (layer "F.Cu") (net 21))
 (segment (start 33.88 -129.315) (end 33.88 -124.785) (width 0.2) (layer "F.Cu") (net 2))
 (segment (start 33.67 -129.987) (end 33.67 -129.525) (width 0.2) (layer "F.Cu") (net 2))
 (segment (start 33.67 -129.525) (end 33.88 -129.315) (width 0.2) (layer "F.Cu") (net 2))
 (segment (start 44.2965 -135.889) (end 44.196 -135.7885) (width 0.2) (layer "F.Cu") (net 22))
 (segment (start 45.72 -135.889) (end 44.2965 -135.889) (width 0.2) (layer "F.Cu") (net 22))
 (segment (start 41.006 -129.779) (end 40.64 -129.413) (width 0.2) (layer "F.Cu") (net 8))
 (segment (start 45.72 -128.143) (end 45.847 -128.016) (width 0.2) (layer "F.Cu") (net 8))
 (segment (start 40.64 -129.413) (end 40.64 -128.651) (width 0.2) (layer "F.Cu") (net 8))
 (segment (start 45.88 -127.983) (end 45.88 -124.785) (width 0.2) (layer "F.Cu") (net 8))
 (segment (start 45.847 -128.016) (end 45.88 -127.983) (width 0.2) (layer "F.Cu") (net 8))
 (segment (start 40.64 -128.651) (end 41.148 -128.143) (width 0.2) (layer "F.Cu") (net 8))
 (segment (start 41.148 -128.143) (end 45.72 -128.143) (width 0.2) (layer "F.Cu") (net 8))
 (segment (start 41.006 -129.987) (end 41.006 -129.779) (width 0.2) (layer "F.Cu") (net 8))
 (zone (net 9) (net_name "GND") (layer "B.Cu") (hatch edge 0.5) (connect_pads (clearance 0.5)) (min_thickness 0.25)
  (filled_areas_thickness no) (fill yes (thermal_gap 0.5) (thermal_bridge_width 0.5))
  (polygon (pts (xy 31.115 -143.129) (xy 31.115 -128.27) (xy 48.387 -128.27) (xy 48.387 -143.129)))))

